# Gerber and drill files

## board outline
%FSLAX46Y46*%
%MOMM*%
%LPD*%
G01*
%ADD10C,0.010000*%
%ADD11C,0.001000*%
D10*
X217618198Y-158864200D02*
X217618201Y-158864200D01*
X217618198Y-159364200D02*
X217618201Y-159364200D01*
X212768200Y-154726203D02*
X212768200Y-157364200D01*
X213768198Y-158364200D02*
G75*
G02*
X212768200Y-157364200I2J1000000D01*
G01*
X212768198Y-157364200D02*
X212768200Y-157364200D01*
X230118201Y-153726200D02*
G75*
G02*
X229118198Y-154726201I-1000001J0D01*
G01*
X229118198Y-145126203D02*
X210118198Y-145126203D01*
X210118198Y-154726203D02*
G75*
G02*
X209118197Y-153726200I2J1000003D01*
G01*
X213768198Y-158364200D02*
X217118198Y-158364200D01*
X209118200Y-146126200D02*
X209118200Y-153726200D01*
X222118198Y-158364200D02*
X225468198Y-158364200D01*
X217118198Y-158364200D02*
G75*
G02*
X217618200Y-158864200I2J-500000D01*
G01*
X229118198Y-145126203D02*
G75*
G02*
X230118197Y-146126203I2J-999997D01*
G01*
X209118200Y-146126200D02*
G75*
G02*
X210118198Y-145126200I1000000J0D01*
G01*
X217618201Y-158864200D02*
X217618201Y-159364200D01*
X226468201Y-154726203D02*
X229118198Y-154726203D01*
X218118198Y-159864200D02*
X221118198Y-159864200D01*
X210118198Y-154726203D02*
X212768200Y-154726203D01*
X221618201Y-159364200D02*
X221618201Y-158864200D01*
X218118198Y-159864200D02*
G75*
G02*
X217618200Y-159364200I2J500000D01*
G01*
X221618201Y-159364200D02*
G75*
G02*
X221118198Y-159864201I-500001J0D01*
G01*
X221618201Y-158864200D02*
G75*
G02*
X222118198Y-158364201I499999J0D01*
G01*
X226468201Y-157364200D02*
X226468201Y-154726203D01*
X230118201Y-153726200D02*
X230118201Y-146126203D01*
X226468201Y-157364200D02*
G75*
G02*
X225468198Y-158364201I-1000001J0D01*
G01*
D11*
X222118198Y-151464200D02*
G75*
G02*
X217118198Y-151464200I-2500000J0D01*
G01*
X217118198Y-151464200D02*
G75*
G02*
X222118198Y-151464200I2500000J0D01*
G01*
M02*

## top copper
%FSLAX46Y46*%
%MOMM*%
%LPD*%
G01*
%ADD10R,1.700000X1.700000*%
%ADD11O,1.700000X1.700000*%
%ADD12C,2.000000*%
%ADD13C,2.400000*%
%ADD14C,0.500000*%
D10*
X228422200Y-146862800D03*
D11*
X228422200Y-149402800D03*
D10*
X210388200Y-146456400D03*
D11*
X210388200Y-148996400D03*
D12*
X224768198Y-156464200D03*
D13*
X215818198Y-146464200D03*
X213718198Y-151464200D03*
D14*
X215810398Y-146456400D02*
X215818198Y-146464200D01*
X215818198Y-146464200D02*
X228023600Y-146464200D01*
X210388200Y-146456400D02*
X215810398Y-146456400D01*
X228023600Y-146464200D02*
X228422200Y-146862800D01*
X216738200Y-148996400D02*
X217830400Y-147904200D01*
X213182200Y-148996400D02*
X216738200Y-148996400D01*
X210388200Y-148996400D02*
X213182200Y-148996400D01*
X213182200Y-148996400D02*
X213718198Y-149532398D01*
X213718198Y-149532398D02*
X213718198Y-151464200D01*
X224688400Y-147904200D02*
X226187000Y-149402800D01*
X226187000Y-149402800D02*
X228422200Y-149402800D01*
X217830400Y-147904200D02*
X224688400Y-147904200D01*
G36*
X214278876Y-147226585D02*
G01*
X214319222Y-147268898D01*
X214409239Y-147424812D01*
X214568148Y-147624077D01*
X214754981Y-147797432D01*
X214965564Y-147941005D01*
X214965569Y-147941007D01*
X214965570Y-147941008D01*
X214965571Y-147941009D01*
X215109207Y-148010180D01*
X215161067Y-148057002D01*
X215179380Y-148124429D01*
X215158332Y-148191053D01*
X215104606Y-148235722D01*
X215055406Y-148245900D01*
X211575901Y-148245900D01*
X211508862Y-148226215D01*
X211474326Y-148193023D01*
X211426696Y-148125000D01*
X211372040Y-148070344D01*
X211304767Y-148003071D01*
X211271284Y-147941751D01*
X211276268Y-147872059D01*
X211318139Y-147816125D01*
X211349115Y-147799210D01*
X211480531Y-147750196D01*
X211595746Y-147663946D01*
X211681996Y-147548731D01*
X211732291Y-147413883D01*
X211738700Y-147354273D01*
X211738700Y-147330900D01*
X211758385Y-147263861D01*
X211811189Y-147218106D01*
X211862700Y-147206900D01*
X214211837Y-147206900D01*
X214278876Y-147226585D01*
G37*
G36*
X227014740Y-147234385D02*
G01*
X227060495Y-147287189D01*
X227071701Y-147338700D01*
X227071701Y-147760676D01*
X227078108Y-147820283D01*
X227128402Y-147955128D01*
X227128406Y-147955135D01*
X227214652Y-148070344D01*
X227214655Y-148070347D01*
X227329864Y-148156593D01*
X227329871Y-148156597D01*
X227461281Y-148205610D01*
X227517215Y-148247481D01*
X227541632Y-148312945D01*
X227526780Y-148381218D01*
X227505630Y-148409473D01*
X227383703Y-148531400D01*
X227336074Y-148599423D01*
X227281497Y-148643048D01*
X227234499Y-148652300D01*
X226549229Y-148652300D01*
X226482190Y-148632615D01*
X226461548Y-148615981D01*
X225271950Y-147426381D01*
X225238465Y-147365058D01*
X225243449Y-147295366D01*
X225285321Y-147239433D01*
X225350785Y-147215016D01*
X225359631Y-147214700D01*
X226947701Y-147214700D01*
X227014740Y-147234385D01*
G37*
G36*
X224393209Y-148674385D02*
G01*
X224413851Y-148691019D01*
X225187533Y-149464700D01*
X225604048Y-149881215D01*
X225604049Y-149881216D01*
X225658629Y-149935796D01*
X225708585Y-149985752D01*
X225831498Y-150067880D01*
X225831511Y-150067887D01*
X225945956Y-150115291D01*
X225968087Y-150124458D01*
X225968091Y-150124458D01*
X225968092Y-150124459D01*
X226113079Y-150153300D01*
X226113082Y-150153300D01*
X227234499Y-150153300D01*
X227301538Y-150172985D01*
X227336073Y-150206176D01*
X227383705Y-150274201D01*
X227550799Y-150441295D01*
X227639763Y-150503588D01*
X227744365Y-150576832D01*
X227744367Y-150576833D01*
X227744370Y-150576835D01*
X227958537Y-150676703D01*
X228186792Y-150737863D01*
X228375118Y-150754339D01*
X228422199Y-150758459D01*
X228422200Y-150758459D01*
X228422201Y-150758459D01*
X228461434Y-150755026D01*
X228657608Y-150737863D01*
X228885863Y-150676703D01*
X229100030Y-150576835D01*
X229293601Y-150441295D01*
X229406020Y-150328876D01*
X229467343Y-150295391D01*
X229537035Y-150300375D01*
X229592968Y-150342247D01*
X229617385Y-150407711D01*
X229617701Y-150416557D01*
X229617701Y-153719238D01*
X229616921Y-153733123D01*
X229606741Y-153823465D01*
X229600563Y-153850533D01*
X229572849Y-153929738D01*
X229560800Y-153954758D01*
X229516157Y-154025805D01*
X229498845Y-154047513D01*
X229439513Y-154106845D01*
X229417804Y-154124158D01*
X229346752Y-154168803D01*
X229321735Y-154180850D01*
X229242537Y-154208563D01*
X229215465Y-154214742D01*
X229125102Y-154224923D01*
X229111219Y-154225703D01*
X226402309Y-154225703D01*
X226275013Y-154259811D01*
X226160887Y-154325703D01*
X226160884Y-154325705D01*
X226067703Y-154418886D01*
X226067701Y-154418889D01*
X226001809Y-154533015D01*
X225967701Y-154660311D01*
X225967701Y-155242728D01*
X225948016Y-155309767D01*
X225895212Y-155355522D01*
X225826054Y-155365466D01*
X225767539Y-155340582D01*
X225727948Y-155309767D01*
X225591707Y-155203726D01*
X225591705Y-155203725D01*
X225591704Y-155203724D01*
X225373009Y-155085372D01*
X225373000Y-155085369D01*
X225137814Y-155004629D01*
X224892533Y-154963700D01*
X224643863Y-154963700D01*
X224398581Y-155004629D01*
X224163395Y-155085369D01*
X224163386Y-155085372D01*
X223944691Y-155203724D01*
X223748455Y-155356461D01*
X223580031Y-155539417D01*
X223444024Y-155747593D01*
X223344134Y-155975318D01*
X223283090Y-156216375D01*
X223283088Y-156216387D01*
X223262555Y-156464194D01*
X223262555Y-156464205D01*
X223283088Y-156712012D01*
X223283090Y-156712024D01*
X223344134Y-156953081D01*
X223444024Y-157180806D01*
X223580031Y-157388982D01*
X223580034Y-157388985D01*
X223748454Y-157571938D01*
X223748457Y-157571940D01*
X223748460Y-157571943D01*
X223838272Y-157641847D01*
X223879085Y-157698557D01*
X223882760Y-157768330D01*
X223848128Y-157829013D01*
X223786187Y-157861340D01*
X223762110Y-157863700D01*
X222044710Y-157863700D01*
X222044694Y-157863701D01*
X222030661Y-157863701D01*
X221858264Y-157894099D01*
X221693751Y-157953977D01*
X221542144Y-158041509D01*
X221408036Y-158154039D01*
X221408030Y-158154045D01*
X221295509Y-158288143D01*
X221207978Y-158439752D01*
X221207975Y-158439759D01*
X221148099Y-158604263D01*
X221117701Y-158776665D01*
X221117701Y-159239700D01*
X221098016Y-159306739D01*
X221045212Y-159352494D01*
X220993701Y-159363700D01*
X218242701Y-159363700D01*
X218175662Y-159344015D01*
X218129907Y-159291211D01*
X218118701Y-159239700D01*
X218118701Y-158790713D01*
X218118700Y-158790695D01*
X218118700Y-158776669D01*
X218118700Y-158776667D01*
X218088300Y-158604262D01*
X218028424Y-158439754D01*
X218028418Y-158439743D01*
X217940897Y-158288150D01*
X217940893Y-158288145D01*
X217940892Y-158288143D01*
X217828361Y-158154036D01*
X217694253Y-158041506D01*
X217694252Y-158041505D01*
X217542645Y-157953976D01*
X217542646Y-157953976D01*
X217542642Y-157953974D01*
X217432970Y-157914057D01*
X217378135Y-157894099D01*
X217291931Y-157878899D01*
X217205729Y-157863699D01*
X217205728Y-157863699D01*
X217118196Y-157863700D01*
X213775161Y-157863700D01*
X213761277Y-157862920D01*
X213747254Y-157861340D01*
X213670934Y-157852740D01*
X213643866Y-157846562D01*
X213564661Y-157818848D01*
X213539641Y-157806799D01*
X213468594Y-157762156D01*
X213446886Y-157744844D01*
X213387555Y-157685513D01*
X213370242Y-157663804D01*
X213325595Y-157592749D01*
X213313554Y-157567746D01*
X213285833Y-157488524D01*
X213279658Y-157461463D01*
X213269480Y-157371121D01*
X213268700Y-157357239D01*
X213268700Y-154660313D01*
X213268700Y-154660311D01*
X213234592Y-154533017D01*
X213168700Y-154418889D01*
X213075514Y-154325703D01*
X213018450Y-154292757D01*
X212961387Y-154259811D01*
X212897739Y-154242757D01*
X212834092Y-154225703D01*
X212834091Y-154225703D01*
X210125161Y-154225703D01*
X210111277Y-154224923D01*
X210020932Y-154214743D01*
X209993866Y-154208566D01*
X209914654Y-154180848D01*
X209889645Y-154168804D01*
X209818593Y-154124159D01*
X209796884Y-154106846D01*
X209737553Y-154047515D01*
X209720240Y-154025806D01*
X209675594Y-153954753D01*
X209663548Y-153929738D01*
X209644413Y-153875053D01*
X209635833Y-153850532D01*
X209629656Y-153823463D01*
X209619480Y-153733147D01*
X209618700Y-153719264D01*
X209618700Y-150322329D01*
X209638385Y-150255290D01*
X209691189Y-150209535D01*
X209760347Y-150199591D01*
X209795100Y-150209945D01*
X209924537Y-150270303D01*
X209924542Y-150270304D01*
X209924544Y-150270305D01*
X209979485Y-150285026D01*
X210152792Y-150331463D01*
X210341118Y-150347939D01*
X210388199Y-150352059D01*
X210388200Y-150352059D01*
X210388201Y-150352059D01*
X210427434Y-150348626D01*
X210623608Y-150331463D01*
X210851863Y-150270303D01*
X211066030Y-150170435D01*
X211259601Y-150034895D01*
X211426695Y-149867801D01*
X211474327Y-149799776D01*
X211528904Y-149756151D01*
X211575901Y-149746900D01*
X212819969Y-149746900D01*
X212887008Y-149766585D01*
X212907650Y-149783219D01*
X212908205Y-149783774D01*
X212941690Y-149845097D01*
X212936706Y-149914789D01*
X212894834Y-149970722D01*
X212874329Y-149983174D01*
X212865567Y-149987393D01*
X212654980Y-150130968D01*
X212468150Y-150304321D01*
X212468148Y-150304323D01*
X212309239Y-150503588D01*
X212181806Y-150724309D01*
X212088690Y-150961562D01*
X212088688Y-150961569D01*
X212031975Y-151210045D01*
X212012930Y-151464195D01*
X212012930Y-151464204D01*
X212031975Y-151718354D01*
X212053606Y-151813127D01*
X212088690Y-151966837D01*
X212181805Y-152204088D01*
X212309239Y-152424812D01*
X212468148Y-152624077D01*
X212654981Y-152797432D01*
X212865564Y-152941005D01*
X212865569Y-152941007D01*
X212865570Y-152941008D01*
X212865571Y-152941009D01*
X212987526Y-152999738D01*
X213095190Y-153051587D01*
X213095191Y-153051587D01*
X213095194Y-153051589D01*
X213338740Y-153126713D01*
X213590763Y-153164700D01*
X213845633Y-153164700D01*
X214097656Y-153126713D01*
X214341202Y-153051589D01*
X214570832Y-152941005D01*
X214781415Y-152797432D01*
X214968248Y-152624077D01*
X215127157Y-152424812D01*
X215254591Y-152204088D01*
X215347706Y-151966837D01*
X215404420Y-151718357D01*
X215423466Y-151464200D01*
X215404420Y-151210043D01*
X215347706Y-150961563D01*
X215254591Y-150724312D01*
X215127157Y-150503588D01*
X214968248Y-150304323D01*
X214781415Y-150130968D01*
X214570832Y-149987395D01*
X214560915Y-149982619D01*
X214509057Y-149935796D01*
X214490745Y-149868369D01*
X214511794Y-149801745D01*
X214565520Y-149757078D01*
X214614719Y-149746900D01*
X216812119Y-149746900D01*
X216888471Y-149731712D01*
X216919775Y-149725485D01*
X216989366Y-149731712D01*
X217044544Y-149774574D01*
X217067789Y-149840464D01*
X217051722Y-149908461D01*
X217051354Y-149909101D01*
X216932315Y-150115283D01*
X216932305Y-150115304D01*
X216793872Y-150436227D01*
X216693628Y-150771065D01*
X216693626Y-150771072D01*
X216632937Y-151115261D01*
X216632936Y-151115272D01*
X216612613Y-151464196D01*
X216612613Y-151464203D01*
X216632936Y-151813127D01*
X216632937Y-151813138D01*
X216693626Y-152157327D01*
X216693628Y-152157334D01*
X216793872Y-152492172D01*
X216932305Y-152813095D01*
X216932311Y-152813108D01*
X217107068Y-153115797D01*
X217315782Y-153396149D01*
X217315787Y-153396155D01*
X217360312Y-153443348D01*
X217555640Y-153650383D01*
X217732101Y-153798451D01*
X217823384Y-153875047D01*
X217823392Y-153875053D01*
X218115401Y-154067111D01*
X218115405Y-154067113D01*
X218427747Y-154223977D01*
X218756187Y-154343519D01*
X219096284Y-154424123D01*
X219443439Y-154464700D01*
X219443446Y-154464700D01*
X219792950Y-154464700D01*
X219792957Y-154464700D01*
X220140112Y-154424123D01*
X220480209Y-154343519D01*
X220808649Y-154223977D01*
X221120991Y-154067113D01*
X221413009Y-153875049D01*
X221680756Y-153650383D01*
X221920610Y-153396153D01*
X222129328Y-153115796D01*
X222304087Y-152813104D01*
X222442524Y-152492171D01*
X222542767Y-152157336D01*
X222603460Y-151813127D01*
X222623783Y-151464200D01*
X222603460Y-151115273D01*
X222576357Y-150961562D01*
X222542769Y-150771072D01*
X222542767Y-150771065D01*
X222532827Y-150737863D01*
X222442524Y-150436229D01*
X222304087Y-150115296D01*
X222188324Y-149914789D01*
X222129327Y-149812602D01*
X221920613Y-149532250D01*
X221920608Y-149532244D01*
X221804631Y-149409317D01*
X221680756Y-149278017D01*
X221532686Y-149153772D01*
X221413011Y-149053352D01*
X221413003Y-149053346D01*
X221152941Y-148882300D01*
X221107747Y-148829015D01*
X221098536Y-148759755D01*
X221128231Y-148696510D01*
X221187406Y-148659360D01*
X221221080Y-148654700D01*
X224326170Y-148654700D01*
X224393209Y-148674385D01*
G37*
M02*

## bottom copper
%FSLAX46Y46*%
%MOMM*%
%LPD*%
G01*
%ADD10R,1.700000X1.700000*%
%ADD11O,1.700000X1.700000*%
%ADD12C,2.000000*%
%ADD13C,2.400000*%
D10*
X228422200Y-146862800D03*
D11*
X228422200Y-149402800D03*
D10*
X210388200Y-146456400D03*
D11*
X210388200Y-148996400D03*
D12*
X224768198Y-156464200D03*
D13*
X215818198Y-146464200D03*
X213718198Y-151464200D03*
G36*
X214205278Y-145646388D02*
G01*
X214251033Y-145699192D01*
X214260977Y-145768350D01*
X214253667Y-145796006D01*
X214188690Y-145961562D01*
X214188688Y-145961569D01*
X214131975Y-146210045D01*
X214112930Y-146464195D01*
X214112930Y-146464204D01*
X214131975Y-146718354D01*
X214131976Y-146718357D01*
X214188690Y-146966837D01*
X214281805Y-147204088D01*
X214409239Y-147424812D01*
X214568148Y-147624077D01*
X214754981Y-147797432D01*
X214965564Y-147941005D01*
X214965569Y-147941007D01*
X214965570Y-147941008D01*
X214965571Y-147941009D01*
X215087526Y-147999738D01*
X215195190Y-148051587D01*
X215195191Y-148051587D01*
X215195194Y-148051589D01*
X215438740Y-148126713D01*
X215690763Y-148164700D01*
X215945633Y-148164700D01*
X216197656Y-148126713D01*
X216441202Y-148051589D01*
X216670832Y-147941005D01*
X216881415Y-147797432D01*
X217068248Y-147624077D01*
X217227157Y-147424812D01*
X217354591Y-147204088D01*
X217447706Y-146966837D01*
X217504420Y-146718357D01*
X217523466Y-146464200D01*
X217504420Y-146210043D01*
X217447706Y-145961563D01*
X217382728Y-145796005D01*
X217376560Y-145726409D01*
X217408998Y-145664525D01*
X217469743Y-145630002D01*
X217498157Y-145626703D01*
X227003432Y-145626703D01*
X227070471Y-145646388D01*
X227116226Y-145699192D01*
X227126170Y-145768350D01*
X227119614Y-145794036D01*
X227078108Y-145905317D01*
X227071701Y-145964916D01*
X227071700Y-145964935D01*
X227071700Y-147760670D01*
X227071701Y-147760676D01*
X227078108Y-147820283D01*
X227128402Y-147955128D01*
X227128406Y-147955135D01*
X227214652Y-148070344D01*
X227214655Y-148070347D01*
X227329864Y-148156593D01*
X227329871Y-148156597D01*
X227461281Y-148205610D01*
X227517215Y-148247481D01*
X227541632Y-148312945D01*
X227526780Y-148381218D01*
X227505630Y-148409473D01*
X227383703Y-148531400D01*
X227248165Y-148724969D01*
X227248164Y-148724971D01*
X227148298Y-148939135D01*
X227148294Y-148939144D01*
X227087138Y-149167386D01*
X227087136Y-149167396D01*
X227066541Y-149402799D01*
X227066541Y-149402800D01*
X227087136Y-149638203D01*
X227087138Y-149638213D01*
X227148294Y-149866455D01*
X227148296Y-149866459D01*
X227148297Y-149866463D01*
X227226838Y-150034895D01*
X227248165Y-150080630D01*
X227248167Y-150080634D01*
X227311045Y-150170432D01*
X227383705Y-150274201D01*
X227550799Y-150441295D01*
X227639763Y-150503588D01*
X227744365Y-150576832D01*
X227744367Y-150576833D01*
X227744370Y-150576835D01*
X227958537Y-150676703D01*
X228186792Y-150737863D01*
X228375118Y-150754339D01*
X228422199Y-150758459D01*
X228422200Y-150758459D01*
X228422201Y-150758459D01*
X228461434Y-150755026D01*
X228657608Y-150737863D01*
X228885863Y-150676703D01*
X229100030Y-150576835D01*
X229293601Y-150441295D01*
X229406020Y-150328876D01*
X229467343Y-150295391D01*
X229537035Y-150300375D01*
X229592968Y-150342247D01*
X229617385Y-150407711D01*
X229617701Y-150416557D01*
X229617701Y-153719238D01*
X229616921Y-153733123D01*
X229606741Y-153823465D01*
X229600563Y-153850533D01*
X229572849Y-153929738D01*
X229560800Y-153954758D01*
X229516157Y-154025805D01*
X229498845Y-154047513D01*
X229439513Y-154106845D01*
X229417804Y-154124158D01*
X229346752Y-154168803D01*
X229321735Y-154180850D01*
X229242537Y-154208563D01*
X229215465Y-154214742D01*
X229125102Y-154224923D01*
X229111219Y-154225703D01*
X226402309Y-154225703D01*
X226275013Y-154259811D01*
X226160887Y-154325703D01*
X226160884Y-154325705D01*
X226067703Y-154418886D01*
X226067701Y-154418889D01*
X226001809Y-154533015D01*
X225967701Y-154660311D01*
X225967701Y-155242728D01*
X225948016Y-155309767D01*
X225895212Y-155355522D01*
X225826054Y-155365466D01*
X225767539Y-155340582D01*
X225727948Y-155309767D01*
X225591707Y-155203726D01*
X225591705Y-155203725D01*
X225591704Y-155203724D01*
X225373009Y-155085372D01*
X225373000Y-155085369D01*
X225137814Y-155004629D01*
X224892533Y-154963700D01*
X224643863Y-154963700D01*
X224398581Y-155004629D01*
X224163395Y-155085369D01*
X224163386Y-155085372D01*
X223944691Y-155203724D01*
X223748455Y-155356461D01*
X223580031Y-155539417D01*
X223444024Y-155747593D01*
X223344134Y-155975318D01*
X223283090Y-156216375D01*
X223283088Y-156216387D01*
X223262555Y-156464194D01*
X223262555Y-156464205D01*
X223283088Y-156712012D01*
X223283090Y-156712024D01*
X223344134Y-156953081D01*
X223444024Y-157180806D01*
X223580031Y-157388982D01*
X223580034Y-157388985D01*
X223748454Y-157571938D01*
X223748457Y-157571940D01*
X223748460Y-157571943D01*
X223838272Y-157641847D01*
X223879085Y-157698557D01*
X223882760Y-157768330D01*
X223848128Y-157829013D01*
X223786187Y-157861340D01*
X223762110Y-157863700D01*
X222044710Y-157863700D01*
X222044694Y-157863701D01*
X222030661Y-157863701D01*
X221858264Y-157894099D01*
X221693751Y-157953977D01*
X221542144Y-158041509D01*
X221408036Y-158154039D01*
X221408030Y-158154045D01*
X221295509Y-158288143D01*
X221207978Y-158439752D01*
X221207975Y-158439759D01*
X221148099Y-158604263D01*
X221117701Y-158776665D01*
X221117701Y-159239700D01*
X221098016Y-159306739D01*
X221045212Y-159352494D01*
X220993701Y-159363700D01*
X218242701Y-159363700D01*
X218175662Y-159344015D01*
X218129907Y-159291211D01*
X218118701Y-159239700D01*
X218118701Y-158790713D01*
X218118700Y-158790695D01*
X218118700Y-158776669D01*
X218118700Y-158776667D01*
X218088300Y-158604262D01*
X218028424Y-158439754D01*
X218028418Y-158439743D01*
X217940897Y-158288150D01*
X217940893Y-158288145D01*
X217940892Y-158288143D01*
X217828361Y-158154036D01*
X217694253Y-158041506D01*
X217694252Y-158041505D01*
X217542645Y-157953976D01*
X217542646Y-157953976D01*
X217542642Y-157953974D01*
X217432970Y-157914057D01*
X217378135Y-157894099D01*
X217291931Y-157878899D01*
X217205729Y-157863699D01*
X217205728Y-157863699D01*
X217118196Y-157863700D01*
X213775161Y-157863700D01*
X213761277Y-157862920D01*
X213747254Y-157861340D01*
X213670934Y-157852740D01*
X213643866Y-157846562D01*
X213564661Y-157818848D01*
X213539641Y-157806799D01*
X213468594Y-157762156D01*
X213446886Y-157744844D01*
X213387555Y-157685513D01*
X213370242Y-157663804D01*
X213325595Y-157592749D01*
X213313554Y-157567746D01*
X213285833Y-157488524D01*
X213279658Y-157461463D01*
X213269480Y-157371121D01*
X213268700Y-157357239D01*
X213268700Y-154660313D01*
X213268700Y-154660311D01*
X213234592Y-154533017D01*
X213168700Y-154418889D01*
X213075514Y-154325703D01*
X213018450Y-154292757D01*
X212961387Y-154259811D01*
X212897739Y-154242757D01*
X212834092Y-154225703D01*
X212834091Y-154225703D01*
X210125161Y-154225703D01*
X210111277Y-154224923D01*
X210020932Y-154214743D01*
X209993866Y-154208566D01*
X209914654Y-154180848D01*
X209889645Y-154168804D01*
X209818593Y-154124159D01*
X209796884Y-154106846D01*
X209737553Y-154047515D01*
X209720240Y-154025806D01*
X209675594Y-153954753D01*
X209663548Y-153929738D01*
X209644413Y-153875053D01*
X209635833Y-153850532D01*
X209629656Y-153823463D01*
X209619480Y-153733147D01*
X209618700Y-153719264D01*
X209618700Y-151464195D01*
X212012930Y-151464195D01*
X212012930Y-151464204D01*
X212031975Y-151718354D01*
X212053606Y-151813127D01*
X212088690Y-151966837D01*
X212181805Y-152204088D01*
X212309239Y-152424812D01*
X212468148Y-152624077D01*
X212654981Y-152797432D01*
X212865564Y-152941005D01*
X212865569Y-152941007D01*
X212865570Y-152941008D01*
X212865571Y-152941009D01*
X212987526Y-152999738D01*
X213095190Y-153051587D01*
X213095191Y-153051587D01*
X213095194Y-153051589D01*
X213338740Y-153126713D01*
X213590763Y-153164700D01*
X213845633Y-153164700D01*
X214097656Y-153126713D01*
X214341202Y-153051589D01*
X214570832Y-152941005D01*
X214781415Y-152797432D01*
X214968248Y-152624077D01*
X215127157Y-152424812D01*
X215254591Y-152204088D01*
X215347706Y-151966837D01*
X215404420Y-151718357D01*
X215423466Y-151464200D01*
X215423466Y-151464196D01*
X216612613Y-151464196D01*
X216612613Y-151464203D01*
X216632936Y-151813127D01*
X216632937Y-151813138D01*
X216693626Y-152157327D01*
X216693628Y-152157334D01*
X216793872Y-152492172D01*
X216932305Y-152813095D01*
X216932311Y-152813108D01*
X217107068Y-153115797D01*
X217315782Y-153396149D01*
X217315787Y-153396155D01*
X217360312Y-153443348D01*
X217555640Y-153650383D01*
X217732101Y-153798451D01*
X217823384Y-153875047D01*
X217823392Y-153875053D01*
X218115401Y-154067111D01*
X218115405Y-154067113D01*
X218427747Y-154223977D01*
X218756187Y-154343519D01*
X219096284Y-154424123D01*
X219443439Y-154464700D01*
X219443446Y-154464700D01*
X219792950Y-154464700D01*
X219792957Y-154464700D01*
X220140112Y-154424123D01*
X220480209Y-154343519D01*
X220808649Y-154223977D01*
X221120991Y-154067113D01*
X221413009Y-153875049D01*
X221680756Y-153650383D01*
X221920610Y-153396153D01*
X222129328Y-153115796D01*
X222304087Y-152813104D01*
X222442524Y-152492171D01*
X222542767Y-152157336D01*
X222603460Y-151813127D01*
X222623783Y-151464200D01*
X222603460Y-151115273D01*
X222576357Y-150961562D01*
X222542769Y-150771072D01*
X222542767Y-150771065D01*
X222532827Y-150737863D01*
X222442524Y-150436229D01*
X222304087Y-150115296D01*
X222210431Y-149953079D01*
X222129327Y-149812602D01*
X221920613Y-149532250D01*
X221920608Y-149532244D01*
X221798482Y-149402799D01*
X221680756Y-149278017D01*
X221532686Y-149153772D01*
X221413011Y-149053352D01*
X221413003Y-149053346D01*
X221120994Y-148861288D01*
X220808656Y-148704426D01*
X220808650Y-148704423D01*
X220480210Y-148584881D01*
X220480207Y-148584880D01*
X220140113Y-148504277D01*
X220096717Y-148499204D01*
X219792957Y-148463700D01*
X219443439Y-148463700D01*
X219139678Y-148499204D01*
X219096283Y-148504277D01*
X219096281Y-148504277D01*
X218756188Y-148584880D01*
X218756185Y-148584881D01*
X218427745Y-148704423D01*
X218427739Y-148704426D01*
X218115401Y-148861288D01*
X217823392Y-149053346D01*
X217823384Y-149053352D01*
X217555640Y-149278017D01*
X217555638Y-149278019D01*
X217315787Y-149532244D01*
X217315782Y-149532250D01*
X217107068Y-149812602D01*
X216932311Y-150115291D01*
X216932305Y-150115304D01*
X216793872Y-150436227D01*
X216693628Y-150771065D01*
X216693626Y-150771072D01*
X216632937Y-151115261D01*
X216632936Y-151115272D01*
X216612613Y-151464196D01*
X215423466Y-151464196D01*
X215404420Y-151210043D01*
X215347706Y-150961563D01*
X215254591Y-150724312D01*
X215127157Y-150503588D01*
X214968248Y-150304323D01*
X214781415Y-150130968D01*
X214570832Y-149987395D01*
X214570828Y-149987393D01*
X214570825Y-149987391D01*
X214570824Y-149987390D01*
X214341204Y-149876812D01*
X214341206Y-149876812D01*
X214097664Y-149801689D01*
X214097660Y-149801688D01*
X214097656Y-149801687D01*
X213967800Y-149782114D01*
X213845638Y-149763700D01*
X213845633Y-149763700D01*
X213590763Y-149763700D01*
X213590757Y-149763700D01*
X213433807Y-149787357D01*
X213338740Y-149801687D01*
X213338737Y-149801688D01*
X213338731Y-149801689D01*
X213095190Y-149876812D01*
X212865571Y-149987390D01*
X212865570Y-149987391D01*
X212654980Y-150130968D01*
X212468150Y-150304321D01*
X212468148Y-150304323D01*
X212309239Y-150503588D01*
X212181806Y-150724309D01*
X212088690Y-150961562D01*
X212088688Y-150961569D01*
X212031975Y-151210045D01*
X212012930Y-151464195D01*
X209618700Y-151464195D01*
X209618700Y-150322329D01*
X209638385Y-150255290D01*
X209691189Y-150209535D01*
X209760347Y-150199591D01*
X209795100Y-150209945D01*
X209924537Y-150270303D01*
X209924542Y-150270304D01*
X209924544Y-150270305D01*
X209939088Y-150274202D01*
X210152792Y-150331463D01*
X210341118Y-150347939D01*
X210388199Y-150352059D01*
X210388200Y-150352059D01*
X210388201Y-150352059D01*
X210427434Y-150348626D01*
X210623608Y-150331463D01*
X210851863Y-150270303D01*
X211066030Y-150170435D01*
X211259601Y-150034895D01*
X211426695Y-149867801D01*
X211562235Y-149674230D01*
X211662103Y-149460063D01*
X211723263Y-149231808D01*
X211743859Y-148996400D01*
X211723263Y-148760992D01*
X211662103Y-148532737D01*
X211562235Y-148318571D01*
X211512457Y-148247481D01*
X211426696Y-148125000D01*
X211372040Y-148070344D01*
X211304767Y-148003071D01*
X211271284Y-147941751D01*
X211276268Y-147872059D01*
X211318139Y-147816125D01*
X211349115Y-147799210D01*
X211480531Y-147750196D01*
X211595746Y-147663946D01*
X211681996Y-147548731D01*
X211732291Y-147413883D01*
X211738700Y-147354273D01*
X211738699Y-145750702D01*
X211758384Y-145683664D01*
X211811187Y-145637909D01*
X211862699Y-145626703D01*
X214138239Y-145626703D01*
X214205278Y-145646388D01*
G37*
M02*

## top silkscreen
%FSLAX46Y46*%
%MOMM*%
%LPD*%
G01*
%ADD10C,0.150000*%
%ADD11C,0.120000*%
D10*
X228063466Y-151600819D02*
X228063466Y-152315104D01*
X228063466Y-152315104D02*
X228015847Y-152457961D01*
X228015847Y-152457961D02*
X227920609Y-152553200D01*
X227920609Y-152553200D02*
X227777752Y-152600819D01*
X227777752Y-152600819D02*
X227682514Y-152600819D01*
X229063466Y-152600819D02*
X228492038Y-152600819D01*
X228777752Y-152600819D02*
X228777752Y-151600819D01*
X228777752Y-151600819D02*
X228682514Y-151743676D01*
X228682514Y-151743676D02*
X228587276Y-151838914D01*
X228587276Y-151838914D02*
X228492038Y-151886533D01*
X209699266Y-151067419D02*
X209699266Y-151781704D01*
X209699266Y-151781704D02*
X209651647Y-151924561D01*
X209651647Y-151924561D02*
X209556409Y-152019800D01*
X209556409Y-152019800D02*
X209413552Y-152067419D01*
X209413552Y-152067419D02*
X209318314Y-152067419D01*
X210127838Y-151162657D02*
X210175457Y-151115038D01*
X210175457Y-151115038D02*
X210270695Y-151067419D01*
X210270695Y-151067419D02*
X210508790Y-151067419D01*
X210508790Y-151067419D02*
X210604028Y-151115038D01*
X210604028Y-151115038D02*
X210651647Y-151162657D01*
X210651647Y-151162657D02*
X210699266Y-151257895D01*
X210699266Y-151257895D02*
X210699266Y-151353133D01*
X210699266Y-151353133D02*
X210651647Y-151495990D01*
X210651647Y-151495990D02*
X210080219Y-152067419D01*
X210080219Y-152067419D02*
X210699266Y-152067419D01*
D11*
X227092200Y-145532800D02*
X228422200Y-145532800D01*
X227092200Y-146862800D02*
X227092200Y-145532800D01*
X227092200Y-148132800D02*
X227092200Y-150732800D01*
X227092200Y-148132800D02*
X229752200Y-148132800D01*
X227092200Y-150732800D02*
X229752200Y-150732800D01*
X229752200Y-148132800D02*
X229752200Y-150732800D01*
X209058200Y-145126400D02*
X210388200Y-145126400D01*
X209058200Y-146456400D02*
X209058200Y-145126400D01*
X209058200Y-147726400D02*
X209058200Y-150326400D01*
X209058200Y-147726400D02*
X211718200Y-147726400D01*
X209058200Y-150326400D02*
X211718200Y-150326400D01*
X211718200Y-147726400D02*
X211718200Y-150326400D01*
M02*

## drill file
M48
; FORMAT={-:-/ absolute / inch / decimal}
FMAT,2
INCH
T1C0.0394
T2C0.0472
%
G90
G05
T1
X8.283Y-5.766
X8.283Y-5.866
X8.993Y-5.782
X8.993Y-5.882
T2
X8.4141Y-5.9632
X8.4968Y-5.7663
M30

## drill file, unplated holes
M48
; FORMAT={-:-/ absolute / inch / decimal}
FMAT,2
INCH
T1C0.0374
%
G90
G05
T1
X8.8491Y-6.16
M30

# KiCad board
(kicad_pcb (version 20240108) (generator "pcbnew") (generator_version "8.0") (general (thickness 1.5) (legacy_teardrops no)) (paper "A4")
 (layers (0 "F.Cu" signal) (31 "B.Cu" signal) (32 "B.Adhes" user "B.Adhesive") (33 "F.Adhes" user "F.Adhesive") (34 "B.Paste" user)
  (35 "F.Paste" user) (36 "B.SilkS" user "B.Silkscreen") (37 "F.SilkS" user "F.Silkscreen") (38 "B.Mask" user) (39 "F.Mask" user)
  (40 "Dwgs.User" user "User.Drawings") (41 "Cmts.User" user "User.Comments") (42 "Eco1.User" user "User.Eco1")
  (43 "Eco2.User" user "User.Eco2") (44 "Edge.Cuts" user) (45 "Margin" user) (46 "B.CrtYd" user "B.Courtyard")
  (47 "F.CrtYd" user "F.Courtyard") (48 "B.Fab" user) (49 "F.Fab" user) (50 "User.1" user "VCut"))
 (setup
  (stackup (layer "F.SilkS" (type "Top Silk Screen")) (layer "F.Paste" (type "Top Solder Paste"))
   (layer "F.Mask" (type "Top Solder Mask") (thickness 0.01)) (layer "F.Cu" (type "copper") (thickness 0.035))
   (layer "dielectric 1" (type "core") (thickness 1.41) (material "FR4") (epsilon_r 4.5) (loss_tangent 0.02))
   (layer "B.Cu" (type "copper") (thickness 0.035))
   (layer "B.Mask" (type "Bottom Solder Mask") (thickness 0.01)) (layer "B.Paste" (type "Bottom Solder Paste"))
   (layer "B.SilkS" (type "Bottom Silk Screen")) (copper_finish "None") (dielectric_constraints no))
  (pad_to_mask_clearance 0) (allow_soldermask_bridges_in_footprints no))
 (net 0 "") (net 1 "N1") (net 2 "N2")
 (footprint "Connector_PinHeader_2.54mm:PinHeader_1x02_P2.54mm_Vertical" (layer "F.Cu") (at 228.4222 146.8628)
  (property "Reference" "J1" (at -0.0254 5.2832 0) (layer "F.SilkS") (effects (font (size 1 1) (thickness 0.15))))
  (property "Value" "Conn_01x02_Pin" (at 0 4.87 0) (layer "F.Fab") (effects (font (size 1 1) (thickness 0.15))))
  (fp_line (start -1.33 -1.33) (end 0 -1.33) (stroke (width 0.12) (type solid)) (layer "F.SilkS"))
  (fp_line (start -1.33 0) (end -1.33 -1.33) (stroke (width 0.12) (type solid)) (layer "F.SilkS"))
  (fp_line (start -1.33 1.27) (end -1.33 3.87) (stroke (width 0.12) (type solid)) (layer "F.SilkS"))
  (fp_line (start -1.33 1.27) (end 1.33 1.27) (stroke (width 0.12) (type solid)) (layer "F.SilkS"))
  (fp_line (start -1.33 3.87) (end 1.33 3.87) (stroke (width 0.12) (type solid)) (layer "F.SilkS"))
  (fp_line (start 1.33 1.27) (end 1.33 3.87) (stroke (width 0.12) (type solid)) (layer "F.SilkS"))
  (pad "1" thru_hole rect (at 0 0) (size 1.7 1.7) (drill 1) (layers "*.Cu" "*.Mask") (remove_unused_layers no) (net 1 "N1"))
  (pad "2" thru_hole oval (at 0 2.54) (size 1.7 1.7) (drill 1) (layers "*.Cu" "*.Mask") (remove_unused_layers no) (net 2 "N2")))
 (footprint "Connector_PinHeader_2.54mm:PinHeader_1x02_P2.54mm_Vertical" (layer "F.Cu") (at 210.3882 146.4564)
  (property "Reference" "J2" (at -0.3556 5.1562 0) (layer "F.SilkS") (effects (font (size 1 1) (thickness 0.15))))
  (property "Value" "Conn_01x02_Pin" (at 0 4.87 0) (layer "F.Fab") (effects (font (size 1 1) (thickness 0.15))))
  (fp_line (start -1.33 -1.33) (end 0 -1.33) (stroke (width 0.12) (type solid)) (layer "F.SilkS"))
  (fp_line (start -1.33 0) (end -1.33 -1.33) (stroke (width 0.12) (type solid)) (layer "F.SilkS"))
  (fp_line (start -1.33 1.27) (end -1.33 3.87) (stroke (width 0.12) (type solid)) (layer "F.SilkS"))
  (fp_line (start -1.33 1.27) (end 1.33 1.27) (stroke (width 0.12) (type solid)) (layer "F.SilkS"))
  (fp_line (start -1.33 3.87) (end 1.33 3.87) (stroke (width 0.12) (type solid)) (layer "F.SilkS"))
  (fp_line (start 1.33 1.27) (end 1.33 3.87) (stroke (width 0.12) (type solid)) (layer "F.SilkS"))
  (pad "1" thru_hole rect (at 0 0) (size 1.7 1.7) (drill 1) (layers "*.Cu" "*.Mask") (remove_unused_layers no) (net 1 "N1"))
  (pad "2" thru_hole oval (at 0 2.54) (size 1.7 1.7) (drill 1) (layers "*.Cu" "*.Mask") (remove_unused_layers no) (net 2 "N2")))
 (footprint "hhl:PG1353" (layer "F.Cu") (at 219.618198 151.4642)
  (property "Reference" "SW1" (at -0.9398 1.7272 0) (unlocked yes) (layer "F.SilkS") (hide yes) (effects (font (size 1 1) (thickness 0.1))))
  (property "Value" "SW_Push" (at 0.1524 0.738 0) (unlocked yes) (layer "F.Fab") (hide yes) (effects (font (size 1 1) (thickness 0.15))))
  (fp_circle (center 0 0) (end 2.5 0) (stroke (width 0.001) (type default)) (fill none) (layer "Edge.Cuts"))
  (pad "" np_thru_hole circle (at 5.15 5) (size 2 2) (drill 0.95) (layers "F&B.Cu" "*.Mask"))
  (pad "1" thru_hole circle (at -3.8 -5) (size 2.4 2.4) (drill 1.2) (layers "*.Cu" "*.Mask") (remove_unused_layers no) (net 1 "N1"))
  (pad "2" thru_hole circle (at -5.9 0) (size 2.4 2.4) (drill 1.2) (layers "*.Cu" "*.Mask") (remove_unused_layers no) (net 2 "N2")))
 (gr_line (start 217.618198 158.8642) (end 217.618201 158.8642) (stroke (width 0.01) (type default)) (layer "Edge.Cuts"))
 (gr_line (start 217.618198 159.3642) (end 217.618201 159.3642) (stroke (width 0.01) (type default)) (layer "Edge.Cuts"))
 (gr_line (start 212.7682 154.726203) (end 212.7682 157.3642) (stroke (width 0.01) (type default)) (layer "Edge.Cuts"))
 (gr_arc (start 213.768198 158.3642) (mid 213.061091 158.071307) (end 212.768198 157.3642) (stroke (width 0.01) (type default))
  (layer "Edge.Cuts"))
 (gr_line (start 212.768198 157.3642) (end 212.7682 157.3642) (stroke (width 0.01) (type default)) (layer "Edge.Cuts"))
 (gr_arc (start 230.118201 153.7262) (mid 229.825307 154.433309) (end 229.118198 154.726203) (stroke (width 0.01) (type default))
  (layer "Edge.Cuts"))
 (gr_line (start 229.118198 145.126203) (end 210.118198 145.126203) (stroke (width 0.01) (type default)) (layer "Edge.Cuts"))
 (gr_arc (start 210.118198 154.726203) (mid 209.411089 154.433309) (end 209.1182 153.7262) (stroke (width 0.01) (type default))
  (layer "Edge.Cuts"))
 (gr_line (start 213.768198 158.3642) (end 217.118198 158.3642) (stroke (width 0.01) (type default)) (layer "Edge.Cuts"))
 (gr_line (start 209.1182 146.1262) (end 209.1182 153.7262) (stroke (width 0.01) (type default)) (layer "Edge.Cuts"))
 (gr_line (start 222.118198 158.3642) (end 225.468198 158.3642) (stroke (width 0.01) (type default)) (layer "Edge.Cuts"))
 (gr_arc (start 217.118198 158.3642) (mid 217.471751 158.510647) (end 217.618198 158.8642) (stroke (width 0.01) (type default))
  (layer "Edge.Cuts"))
 (gr_arc (start 229.118198 145.126203) (mid 229.825304 145.419096) (end 230.118201 146.126203) (stroke (width 0.01) (type default))
  (layer "Edge.Cuts"))
 (gr_arc (start 209.1182 146.1262) (mid 209.411093 145.419095) (end 210.118198 145.126203) (stroke (width 0.01) (type default))
  (layer "Edge.Cuts"))
 (gr_line (start 217.618201 158.8642) (end 217.618201 159.3642) (stroke (width 0.01) (type default)) (layer "Edge.Cuts"))
 (gr_line (start 226.468201 154.726203) (end 229.118198 154.726203) (stroke (width 0.01) (type default)) (layer "Edge.Cuts"))
 (gr_line (start 218.118198 159.8642) (end 221.118198 159.8642) (stroke (width 0.01) (type default)) (layer "Edge.Cuts"))
 (gr_line (start 210.118198 154.726203) (end 212.7682 154.726203) (stroke (width 0.01) (type default)) (layer "Edge.Cuts"))
 (gr_line (start 221.618201 159.3642) (end 221.618201 158.8642) (stroke (width 0.01) (type default)) (layer "Edge.Cuts"))
 (gr_arc (start 218.118198 159.8642) (mid 217.764645 159.717753) (end 217.618198 159.3642) (stroke (width 0.01) (type default))
  (layer "Edge.Cuts"))
 (gr_arc (start 221.618201 159.3642) (mid 221.471754 159.717756) (end 221.118198 159.8642) (stroke (width 0.01) (type default))
  (layer "Edge.Cuts"))
 (gr_arc (start 221.618201 158.8642) (mid 221.764647 158.510649) (end 222.118198 158.3642) (stroke (width 0.01) (type default))
  (layer "Edge.Cuts"))
 (gr_line (start 226.468201 157.3642) (end 226.468201 154.726203) (stroke (width 0.01) (type default)) (layer "Edge.Cuts"))
 (gr_line (start 230.118201 153.7262) (end 230.118201 146.126203) (stroke (width 0.01) (type default)) (layer "Edge.Cuts"))
 (gr_arc (start 226.468201 157.3642) (mid 226.175307 158.071309) (end 225.468198 158.3642) (stroke (width 0.01) (type default))
  (layer "Edge.Cuts"))
 (segment (start 215.810398 146.4564) (end 215.818198 146.4642) (width 0.5) (layer "F.Cu") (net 1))
 (segment (start 215.818198 146.4642) (end 228.0236 146.4642) (width 0.5) (layer "F.Cu") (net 1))
 (segment (start 210.3882 146.4564) (end 215.810398 146.4564) (width 0.5) (layer "F.Cu") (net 1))
 (segment (start 228.0236 146.4642) (end 228.4222 146.8628) (width 0.5) (layer "F.Cu") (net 1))
 (segment (start 216.7382 148.9964) (end 217.8304 147.9042) (width 0.5) (layer "F.Cu") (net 2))
 (segment (start 213.1822 148.9964) (end 216.7382 148.9964) (width 0.5) (layer "F.Cu") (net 2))
 (segment (start 210.3882 148.9964) (end 213.1822 148.9964) (width 0.5) (layer "F.Cu") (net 2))
 (segment (start 213.1822 148.9964) (end 213.718198 149.532398) (width 0.5) (layer "F.Cu") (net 2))
 (segment (start 213.718198 149.532398) (end 213.718198 151.4642) (width 0.5) (layer "F.Cu") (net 2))
 (segment (start 224.6884 147.9042) (end 226.187 149.4028) (width 0.5) (layer "F.Cu") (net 2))
 (segment (start 226.187 149.4028) (end 228.4222 149.4028) (width 0.5) (layer "F.Cu") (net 2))
 (segment (start 217.8304 147.9042) (end 224.6884 147.9042) (width 0.5) (layer "F.Cu") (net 2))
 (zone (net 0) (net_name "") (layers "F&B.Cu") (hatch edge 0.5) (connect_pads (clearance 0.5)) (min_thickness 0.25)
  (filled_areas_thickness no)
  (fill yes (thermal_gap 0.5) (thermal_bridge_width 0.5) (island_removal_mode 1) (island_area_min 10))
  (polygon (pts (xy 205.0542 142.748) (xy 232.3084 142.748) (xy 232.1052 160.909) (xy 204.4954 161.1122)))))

